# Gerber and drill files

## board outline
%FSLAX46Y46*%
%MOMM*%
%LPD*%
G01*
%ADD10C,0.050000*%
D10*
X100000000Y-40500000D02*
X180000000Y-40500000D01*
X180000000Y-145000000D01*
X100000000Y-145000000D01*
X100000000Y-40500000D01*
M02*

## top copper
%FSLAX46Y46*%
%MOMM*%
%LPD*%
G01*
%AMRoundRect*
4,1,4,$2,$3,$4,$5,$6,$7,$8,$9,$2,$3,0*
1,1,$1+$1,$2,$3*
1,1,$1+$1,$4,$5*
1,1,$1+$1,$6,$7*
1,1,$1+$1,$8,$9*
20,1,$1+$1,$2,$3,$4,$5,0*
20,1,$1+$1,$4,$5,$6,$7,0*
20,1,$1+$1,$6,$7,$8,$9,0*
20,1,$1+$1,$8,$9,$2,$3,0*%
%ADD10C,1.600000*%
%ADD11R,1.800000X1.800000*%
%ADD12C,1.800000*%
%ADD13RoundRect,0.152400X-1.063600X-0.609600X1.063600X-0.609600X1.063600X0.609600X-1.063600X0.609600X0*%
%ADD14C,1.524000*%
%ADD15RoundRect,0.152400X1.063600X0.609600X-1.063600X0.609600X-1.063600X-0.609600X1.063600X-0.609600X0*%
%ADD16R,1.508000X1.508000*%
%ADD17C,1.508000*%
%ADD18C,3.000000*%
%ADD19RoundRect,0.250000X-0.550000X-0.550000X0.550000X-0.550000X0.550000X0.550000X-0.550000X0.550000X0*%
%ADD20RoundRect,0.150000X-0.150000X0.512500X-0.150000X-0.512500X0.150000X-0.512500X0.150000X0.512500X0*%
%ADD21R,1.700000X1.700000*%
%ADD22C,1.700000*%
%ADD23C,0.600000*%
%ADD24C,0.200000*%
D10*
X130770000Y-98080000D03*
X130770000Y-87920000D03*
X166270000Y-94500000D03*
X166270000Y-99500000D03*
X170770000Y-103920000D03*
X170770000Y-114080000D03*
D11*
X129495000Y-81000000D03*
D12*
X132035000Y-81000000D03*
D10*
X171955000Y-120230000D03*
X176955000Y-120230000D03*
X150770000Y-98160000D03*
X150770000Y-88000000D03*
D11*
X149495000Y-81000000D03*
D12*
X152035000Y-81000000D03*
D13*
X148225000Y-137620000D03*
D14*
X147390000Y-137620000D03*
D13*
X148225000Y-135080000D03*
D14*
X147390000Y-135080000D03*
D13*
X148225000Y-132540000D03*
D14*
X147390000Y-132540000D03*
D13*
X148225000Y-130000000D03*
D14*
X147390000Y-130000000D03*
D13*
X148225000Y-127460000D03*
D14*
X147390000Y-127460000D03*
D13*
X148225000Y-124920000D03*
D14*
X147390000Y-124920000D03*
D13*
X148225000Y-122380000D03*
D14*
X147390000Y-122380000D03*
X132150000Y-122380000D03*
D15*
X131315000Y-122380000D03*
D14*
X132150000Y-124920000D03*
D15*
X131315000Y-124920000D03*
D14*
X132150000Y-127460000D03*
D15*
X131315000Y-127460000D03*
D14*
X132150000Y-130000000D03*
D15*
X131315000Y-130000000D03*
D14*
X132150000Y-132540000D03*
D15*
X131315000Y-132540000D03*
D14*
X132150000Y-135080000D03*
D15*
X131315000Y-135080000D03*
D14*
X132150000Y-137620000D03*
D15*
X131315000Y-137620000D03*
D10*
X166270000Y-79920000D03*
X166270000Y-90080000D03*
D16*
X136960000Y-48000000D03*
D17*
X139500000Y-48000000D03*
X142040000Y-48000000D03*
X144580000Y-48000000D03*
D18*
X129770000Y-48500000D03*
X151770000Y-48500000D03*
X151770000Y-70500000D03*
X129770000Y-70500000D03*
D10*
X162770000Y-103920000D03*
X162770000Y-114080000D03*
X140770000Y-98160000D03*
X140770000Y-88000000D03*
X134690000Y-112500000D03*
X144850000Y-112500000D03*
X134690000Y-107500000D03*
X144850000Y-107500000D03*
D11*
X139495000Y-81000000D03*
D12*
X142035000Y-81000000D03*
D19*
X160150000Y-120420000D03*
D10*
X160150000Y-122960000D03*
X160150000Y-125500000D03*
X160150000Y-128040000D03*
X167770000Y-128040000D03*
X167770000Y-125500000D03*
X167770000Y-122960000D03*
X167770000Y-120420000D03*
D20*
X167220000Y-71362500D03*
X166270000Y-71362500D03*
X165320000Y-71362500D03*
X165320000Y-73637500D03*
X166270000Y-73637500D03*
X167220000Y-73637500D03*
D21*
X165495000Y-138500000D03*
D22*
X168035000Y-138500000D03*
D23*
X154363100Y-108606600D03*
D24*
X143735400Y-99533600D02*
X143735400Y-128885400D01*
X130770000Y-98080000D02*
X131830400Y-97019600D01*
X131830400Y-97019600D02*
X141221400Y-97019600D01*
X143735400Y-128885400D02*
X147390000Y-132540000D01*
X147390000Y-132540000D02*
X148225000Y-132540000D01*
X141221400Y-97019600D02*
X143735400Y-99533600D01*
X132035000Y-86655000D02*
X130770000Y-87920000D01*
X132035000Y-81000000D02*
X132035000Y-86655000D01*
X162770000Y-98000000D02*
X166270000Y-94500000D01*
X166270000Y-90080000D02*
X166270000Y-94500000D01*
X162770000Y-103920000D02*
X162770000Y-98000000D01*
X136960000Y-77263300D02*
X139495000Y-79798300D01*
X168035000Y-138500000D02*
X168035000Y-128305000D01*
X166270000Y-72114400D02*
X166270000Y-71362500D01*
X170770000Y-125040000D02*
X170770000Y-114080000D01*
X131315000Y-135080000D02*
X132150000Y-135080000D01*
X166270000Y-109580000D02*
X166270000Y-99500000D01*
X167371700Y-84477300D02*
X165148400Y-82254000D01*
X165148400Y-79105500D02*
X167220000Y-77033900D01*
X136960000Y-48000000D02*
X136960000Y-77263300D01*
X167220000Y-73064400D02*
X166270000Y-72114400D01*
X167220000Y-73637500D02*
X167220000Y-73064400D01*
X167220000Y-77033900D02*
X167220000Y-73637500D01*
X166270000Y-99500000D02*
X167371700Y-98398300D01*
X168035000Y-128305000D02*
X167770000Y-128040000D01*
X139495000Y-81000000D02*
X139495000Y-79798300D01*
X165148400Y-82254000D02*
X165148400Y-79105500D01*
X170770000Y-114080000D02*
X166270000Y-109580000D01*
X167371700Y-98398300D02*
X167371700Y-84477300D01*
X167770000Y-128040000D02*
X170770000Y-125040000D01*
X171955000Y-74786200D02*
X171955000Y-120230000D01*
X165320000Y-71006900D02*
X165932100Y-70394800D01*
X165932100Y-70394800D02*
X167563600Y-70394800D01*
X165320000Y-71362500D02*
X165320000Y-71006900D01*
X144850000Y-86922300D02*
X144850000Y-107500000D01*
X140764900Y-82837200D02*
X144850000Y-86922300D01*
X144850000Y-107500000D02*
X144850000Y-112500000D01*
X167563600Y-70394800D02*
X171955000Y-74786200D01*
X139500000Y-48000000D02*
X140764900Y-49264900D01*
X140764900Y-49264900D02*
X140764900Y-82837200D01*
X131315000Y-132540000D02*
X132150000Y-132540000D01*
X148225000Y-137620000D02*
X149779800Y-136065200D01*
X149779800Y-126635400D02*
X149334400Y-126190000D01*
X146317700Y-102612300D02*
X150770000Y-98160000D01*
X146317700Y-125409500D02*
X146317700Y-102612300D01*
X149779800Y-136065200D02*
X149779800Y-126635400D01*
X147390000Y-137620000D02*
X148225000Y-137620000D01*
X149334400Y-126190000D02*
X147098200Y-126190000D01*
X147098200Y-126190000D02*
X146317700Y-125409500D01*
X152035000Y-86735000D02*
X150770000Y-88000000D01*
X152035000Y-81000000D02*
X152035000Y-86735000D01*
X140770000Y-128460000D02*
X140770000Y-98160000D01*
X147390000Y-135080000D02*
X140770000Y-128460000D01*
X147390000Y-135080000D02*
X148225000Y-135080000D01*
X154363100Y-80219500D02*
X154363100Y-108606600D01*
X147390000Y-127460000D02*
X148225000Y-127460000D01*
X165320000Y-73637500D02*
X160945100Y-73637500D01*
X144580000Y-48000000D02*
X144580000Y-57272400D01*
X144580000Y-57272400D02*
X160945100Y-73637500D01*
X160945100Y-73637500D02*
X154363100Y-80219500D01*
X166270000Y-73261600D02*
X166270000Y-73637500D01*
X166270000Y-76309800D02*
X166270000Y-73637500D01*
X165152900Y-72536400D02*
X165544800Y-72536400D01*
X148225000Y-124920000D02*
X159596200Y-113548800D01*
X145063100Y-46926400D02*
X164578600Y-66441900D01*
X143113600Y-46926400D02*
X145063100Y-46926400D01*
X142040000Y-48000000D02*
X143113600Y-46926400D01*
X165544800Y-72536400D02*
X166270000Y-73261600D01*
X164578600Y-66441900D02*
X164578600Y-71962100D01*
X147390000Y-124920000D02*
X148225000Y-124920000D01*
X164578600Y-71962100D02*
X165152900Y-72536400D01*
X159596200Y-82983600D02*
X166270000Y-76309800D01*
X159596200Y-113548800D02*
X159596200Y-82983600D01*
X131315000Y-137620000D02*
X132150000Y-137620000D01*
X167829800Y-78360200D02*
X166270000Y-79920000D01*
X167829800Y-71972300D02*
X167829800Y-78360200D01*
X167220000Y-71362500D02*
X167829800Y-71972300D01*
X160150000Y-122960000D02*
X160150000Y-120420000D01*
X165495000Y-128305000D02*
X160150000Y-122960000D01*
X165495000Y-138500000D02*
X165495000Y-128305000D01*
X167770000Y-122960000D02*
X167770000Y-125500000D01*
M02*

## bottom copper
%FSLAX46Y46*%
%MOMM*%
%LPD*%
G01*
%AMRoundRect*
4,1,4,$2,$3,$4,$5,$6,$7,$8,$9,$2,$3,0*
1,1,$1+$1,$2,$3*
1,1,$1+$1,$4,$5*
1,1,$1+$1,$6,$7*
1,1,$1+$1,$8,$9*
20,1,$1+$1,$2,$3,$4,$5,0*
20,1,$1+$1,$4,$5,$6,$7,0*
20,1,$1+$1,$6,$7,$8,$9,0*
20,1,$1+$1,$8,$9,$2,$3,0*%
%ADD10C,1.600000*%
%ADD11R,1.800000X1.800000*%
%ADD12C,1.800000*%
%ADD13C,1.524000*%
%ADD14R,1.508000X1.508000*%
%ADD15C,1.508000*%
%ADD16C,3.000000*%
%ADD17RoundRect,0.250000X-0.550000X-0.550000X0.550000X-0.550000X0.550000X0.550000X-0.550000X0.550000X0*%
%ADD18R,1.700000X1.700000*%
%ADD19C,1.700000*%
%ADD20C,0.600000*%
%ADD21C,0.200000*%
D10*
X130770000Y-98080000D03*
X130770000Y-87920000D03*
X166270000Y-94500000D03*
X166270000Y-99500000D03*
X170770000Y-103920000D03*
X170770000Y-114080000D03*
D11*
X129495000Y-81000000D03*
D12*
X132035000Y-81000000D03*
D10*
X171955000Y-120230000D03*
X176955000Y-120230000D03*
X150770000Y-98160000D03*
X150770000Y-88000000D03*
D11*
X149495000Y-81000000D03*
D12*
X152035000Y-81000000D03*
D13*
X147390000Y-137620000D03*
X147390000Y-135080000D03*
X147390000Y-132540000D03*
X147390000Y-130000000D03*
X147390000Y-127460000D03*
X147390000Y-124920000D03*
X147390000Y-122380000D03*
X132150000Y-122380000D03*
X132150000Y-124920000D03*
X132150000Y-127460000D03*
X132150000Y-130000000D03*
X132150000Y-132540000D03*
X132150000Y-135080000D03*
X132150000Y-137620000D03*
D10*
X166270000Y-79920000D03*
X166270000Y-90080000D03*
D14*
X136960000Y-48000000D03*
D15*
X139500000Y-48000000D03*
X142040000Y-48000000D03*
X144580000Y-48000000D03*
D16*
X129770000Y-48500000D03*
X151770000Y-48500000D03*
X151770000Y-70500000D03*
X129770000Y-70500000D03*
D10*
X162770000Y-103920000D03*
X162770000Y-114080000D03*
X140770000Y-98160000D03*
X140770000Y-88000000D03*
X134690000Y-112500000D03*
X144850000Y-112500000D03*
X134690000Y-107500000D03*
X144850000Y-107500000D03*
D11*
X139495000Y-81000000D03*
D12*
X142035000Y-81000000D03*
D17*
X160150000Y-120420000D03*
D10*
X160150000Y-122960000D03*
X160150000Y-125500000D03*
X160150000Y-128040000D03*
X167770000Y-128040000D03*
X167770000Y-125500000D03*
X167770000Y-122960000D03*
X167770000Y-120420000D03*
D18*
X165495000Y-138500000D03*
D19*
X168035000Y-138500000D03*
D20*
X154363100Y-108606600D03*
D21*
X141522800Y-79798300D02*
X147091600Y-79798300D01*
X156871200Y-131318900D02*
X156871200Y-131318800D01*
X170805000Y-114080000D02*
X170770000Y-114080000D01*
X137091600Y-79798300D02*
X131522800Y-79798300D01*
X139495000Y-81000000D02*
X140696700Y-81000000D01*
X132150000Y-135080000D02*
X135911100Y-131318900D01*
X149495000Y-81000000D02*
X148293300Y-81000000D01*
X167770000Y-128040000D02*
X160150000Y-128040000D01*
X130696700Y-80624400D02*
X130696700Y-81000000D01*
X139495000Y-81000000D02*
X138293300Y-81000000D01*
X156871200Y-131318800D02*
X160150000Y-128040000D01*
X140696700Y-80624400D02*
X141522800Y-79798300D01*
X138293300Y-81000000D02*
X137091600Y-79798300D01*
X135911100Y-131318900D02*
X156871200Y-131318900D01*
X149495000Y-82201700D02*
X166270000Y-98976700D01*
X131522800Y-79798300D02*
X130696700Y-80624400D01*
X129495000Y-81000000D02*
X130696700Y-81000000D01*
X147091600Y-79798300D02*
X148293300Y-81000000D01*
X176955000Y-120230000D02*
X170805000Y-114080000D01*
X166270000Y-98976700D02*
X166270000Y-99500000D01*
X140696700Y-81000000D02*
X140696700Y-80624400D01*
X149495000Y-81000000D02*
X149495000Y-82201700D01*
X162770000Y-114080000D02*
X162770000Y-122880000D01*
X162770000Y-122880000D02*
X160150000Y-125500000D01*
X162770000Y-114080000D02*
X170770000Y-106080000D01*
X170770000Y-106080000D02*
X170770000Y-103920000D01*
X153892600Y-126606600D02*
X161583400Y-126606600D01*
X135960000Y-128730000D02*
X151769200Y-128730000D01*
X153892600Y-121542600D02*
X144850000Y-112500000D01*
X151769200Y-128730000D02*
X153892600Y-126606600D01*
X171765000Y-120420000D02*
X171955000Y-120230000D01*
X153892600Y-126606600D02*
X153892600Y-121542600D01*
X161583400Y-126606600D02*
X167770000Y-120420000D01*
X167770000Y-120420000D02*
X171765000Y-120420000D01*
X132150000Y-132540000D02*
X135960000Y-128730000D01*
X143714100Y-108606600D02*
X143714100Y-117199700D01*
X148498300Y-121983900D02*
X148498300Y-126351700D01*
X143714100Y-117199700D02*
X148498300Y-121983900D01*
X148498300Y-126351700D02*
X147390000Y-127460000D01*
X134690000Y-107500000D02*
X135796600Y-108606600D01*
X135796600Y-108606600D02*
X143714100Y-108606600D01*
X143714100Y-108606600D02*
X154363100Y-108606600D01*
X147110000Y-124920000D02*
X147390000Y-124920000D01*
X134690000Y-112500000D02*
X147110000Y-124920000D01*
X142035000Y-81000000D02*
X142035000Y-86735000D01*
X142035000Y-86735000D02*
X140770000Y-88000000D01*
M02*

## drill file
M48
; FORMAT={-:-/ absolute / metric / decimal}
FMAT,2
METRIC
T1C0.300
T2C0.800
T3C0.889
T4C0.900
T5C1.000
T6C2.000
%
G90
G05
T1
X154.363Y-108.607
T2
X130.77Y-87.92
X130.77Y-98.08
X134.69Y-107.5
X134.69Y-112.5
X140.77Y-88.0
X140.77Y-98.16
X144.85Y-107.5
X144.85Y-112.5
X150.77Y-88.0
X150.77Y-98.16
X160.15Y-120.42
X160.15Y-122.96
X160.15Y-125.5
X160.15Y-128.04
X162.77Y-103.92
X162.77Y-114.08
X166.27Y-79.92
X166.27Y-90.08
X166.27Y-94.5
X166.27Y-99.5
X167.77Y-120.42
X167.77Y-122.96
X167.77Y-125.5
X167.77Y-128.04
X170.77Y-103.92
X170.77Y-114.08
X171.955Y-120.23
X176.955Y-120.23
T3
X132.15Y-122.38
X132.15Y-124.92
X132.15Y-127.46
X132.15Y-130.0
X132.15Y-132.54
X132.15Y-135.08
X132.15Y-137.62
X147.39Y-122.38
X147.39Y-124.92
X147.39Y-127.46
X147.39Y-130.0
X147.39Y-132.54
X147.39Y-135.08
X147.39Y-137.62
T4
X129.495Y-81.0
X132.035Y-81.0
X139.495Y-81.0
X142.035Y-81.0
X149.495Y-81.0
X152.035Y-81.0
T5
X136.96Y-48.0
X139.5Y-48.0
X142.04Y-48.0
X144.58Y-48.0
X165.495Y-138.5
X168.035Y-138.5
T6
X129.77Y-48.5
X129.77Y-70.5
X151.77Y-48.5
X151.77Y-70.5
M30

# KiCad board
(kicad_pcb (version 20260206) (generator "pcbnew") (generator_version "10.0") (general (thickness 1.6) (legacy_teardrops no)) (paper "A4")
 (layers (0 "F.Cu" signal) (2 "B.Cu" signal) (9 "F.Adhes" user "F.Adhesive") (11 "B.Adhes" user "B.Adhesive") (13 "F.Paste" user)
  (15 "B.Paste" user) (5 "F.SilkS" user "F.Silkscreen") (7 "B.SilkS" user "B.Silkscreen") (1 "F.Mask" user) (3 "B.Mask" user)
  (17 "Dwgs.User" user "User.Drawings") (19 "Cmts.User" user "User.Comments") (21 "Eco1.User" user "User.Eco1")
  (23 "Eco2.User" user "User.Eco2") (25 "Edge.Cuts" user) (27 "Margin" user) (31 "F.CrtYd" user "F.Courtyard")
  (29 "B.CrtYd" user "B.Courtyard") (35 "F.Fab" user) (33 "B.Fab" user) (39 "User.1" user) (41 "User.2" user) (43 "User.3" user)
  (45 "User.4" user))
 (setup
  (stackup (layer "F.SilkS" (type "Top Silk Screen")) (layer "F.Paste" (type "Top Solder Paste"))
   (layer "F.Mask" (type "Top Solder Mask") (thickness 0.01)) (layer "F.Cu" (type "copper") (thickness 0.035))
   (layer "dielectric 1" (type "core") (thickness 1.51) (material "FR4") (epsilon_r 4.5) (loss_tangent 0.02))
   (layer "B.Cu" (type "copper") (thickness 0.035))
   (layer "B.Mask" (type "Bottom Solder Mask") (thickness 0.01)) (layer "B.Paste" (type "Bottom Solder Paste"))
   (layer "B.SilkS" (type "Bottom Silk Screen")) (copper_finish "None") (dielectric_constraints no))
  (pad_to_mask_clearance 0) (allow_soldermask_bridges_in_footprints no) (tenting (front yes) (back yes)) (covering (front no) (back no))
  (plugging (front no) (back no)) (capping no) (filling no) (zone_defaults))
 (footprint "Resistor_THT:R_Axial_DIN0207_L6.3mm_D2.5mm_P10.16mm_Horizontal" (layer "F.Cu") (at 130.77 98.08 90)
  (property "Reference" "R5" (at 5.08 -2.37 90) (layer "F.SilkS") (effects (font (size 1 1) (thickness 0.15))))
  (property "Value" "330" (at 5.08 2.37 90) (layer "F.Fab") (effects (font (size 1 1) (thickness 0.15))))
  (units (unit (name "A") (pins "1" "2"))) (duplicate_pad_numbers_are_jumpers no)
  (pad "1" thru_hole circle (at 0 0 90) (size 1.6 1.6) (drill 0.8) (layers "*.Cu" "*.Mask") (remove_unused_layers no) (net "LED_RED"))
  (pad "2" thru_hole circle (at 10.16 0 90) (size 1.6 1.6) (drill 0.8) (layers "*.Cu" "*.Mask") (remove_unused_layers no) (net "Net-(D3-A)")))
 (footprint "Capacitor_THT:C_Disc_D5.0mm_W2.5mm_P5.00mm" (layer "F.Cu") (at 166.27 94.5 -90)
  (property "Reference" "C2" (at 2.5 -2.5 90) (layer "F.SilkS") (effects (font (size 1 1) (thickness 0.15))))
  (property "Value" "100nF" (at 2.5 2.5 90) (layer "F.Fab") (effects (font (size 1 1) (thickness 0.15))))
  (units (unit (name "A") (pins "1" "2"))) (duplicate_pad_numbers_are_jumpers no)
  (pad "1" thru_hole circle (at 0 0 270) (size 1.6 1.6) (drill 0.8) (layers "*.Cu" "*.Mask") (remove_unused_layers no) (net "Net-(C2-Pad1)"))
  (pad "2" thru_hole circle (at 5 0 270) (size 1.6 1.6) (drill 0.8) (layers "*.Cu" "*.Mask") (remove_unused_layers no) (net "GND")))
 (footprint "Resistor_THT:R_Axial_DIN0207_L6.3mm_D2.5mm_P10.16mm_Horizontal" (layer "F.Cu") (at 170.77 103.92 -90)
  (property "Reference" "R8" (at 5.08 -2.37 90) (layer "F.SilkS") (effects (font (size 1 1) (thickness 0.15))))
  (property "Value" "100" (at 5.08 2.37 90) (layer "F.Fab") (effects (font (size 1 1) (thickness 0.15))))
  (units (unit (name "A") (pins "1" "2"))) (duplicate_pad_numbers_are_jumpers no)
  (pad "1" thru_hole circle (at 0 0 270) (size 1.6 1.6) (drill 0.8) (layers "*.Cu" "*.Mask") (remove_unused_layers no) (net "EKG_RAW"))
  (pad "2" thru_hole circle (at 10.16 0 270) (size 1.6 1.6) (drill 0.8) (layers "*.Cu" "*.Mask") (remove_unused_layers no) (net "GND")))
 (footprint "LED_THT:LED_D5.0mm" (layer "F.Cu") (at 129.495 81)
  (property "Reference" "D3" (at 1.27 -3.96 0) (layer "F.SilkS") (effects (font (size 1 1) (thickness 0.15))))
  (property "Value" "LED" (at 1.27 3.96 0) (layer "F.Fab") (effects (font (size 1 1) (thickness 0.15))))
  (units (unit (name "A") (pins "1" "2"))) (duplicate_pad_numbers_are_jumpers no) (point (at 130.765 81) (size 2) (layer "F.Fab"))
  (pad "1" thru_hole rect (at 0 0) (size 1.8 1.8) (drill 0.9) (layers "*.Cu" "*.Mask") (remove_unused_layers no) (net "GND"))
  (pad "2" thru_hole circle (at 2.54 0) (size 1.8 1.8) (drill 0.9) (layers "*.Cu" "*.Mask") (remove_unused_layers no) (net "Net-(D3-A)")))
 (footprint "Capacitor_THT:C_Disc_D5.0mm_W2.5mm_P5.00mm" (layer "F.Cu") (at 171.955 120.23)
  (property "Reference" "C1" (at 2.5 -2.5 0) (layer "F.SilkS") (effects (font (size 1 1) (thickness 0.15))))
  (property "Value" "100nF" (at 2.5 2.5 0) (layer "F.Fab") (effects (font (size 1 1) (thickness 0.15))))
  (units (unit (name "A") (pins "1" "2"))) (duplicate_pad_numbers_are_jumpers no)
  (pad "1" thru_hole circle (at 0 0) (size 1.6 1.6) (drill 0.8) (layers "*.Cu" "*.Mask") (remove_unused_layers no) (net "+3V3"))
  (pad "2" thru_hole circle (at 5 0) (size 1.6 1.6) (drill 0.8) (layers "*.Cu" "*.Mask") (remove_unused_layers no) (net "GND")))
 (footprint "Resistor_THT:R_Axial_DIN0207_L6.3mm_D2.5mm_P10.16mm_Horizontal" (layer "F.Cu") (at 150.77 98.16 90)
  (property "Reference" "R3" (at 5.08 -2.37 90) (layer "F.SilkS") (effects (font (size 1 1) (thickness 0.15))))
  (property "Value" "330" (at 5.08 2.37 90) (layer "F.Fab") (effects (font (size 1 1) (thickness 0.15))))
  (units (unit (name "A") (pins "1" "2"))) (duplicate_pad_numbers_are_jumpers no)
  (pad "1" thru_hole circle (at 0 0 90) (size 1.6 1.6) (drill 0.8) (layers "*.Cu" "*.Mask") (remove_unused_layers no) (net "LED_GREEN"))
  (pad "2" thru_hole circle (at 10.16 0 90) (size 1.6 1.6) (drill 0.8) (layers "*.Cu" "*.Mask") (remove_unused_layers no) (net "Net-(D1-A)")))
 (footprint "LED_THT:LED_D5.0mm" (layer "F.Cu") (at 149.495 81)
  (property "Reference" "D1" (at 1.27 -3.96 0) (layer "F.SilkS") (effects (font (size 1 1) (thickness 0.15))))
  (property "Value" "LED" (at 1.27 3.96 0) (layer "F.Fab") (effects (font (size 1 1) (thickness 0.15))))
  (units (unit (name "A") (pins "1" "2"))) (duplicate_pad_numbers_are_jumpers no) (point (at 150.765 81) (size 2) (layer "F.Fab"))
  (pad "1" thru_hole rect (at 0 0) (size 1.8 1.8) (drill 0.9) (layers "*.Cu" "*.Mask") (remove_unused_layers no) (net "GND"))
  (pad "2" thru_hole circle (at 2.54 0) (size 1.8 1.8) (drill 0.9) (layers "*.Cu" "*.Mask") (remove_unused_layers no) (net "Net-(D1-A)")))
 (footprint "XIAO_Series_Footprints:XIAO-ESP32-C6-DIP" (layer "F.Cu") (at 139.77 130 -90)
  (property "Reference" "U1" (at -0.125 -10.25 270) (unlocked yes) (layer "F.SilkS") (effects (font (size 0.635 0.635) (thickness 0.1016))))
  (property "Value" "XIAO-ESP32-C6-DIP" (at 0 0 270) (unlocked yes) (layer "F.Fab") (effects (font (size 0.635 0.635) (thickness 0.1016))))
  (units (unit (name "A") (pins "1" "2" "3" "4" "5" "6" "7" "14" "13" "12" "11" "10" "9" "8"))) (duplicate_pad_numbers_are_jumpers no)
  (pad "1" smd roundrect (at 7.62 -8.455) (size 2.432 1.524) (layers "F.Cu" "F.Mask") (roundrect_rratio 0.1) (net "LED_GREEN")
   (thermal_bridge_angle 45))
  (pad "1" thru_hole circle (at 7.62 -7.62) (size 1.524 1.524) (drill 0.889) (layers "*.Cu" "*.Mask") (remove_unused_layers no)
   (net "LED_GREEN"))
  (pad "2" smd roundrect (at 5.08 -8.455) (size 2.432 1.524) (layers "F.Cu" "F.Mask") (roundrect_rratio 0.1) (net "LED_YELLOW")
   (thermal_bridge_angle 45))
  (pad "2" thru_hole circle (at 5.08 -7.62) (size 1.524 1.524) (drill 0.889) (layers "*.Cu" "*.Mask") (remove_unused_layers no)
   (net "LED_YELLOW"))
  (pad "3" smd roundrect (at 2.54 -8.455) (size 2.432 1.524) (layers "F.Cu" "F.Mask") (roundrect_rratio 0.1) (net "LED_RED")
   (thermal_bridge_angle 45))
  (pad "3" thru_hole circle (at 2.54 -7.62) (size 1.524 1.524) (drill 0.889) (layers "*.Cu" "*.Mask") (remove_unused_layers no)
   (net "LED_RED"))
  (pad "4" smd roundrect (at 0 -8.455) (size 2.432 1.524) (layers "F.Cu" "F.Mask") (roundrect_rratio 0.1)
   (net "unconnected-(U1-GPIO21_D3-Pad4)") (thermal_bridge_angle 45))
  (pad "4" thru_hole circle (at 0 -7.62) (size 1.524 1.524) (drill 0.889) (layers "*.Cu" "*.Mask") (remove_unused_layers no)
   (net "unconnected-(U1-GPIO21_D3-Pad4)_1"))
  (pad "5" smd roundrect (at -2.54 -8.455) (size 2.432 1.524) (layers "F.Cu" "F.Mask") (roundrect_rratio 0.1) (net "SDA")
   (thermal_bridge_angle 45))
  (pad "5" thru_hole circle (at -2.54 -7.62) (size 1.524 1.524) (drill 0.889) (layers "*.Cu" "*.Mask") (remove_unused_layers no) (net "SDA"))
  (pad "6" smd roundrect (at -5.08 -8.455) (size 2.432 1.524) (layers "F.Cu" "F.Mask") (roundrect_rratio 0.1) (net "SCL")
   (thermal_bridge_angle 45))
  (pad "6" thru_hole circle (at -5.08 -7.62) (size 1.524 1.524) (drill 0.889) (layers "*.Cu" "*.Mask") (remove_unused_layers no) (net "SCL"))
  (pad "7" smd roundrect (at -7.62 -8.455) (size 2.432 1.524) (layers "F.Cu" "F.Mask") (roundrect_rratio 0.1)
   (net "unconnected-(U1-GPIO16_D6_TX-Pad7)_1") (thermal_bridge_angle 45))
  (pad "7" thru_hole circle (at -7.62 -7.62) (size 1.524 1.524) (drill 0.889) (layers "*.Cu" "*.Mask") (remove_unused_layers no)
   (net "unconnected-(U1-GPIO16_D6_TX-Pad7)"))
  (pad "8" thru_hole circle (at -7.62 7.62 180) (size 1.524 1.524) (drill 0.889) (layers "*.Cu" "*.Mask") (remove_unused_layers no)
   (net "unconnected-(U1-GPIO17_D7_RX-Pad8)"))
  (pad "8" smd roundrect (at -7.62 8.455 180) (size 2.432 1.524) (layers "F.Cu" "F.Mask") (roundrect_rratio 0.1)
   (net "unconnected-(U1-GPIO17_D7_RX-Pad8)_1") (thermal_bridge_angle 45))
  (pad "9" thru_hole circle (at -5.08 7.62 180) (size 1.524 1.524) (drill 0.889) (layers "*.Cu" "*.Mask") (remove_unused_layers no)
   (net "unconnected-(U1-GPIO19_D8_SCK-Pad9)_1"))
  (pad "9" smd roundrect (at -5.08 8.455 180) (size 2.432 1.524) (layers "F.Cu" "F.Mask") (roundrect_rratio 0.1)
   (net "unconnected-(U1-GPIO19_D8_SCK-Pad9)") (thermal_bridge_angle 45))
  (pad "10" thru_hole circle (at -2.54 7.62 180) (size 1.524 1.524) (drill 0.889) (layers "*.Cu" "*.Mask") (remove_unused_layers no)
   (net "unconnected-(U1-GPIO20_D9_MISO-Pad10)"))
  (pad "10" smd roundrect (at -2.54 8.455 180) (size 2.432 1.524) (layers "F.Cu" "F.Mask") (roundrect_rratio 0.1)
   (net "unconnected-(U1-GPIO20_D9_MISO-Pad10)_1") (thermal_bridge_angle 45))
  (pad "11" thru_hole circle (at 0 7.62 180) (size 1.524 1.524) (drill 0.889) (layers "*.Cu" "*.Mask") (remove_unused_layers no)
   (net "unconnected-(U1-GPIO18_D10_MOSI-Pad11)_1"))
  (pad "11" smd roundrect (at 0 8.455 180) (size 2.432 1.524) (layers "F.Cu" "F.Mask") (roundrect_rratio 0.1)
   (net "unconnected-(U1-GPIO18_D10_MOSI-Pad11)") (thermal_bridge_angle 45))
  (pad "12" thru_hole circle (at 2.54 7.62 180) (size 1.524 1.524) (drill 0.889) (layers "*.Cu" "*.Mask") (remove_unused_layers no)
   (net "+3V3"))
  (pad "12" smd roundrect (at 2.54 8.455 180) (size 2.432 1.524) (layers "F.Cu" "F.Mask") (roundrect_rratio 0.1) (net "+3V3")
   (thermal_bridge_angle 45))
  (pad "13" thru_hole circle (at 5.08 7.62 180) (size 1.524 1.524) (drill 0.889) (layers "*.Cu" "*.Mask") (remove_unused_layers no)
   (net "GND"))
  (pad "13" smd roundrect (at 5.08 8.455 180) (size 2.432 1.524) (layers "F.Cu" "F.Mask") (roundrect_rratio 0.1) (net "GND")
   (thermal_bridge_angle 45))
  (pad "14" thru_hole circle (at 7.62 7.62 180) (size 1.524 1.524) (drill 0.889) (layers "*.Cu" "*.Mask") (remove_unused_layers no)
   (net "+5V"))
  (pad "14" smd roundrect (at 7.62 8.455 180) (size 2.432 1.524) (layers "F.Cu" "F.Mask") (roundrect_rratio 0.1) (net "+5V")
   (thermal_bridge_angle 45)))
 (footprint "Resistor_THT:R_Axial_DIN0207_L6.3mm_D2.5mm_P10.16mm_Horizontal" (layer "F.Cu") (at 166.27 79.92 -90)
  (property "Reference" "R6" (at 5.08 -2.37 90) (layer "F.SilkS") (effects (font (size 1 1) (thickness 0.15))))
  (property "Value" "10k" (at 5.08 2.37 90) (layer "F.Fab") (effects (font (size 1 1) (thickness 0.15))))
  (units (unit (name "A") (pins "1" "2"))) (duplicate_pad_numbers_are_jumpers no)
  (pad "1" thru_hole circle (at 0 0 270) (size 1.6 1.6) (drill 0.8) (layers "*.Cu" "*.Mask") (remove_unused_layers no) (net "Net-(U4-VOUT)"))
  (pad "2" thru_hole circle (at 10.16 0 270) (size 1.6 1.6) (drill 0.8) (layers "*.Cu" "*.Mask") (remove_unused_layers no)
   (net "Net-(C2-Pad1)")))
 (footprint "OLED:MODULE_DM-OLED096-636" (layer "F.Cu") (at 140.77 59.5)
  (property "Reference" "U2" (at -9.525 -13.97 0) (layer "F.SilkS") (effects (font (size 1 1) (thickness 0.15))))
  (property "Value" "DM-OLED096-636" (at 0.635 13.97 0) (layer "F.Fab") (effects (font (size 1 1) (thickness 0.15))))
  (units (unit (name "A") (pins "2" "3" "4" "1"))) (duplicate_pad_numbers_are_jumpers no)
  (pad "1" thru_hole rect (at -3.81 -11.5) (size 1.508 1.508) (drill 1) (layers "*.Cu" "*.Mask") (remove_unused_layers no) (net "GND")
   (solder_mask_margin 0.102))
  (pad "2" thru_hole circle (at -1.27 -11.5) (size 1.508 1.508) (drill 1) (layers "*.Cu" "*.Mask") (remove_unused_layers no) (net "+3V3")
   (solder_mask_margin 0.102))
  (pad "3" thru_hole circle (at 1.27 -11.5) (size 1.508 1.508) (drill 1) (layers "*.Cu" "*.Mask") (remove_unused_layers no) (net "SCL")
   (solder_mask_margin 0.102))
  (pad "4" thru_hole circle (at 3.81 -11.5) (size 1.508 1.508) (drill 1) (layers "*.Cu" "*.Mask") (remove_unused_layers no) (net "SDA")
   (solder_mask_margin 0.102))
  (pad "S1" thru_hole circle (at -11 -11) (size 3 3) (drill 2) (layers "*.Cu" "*.Mask") (remove_unused_layers no) (solder_mask_margin 0.102))
  (pad "S2" thru_hole circle (at 11 -11) (size 3 3) (drill 2) (layers "*.Cu" "*.Mask") (remove_unused_layers no) (solder_mask_margin 0.102))
  (pad "S3" thru_hole circle (at 11 11) (size 3 3) (drill 2) (layers "*.Cu" "*.Mask") (remove_unused_layers no) (solder_mask_margin 0.102))
  (pad "S4" thru_hole circle (at -11 11) (size 3 3) (drill 2) (layers "*.Cu" "*.Mask") (remove_unused_layers no) (solder_mask_margin 0.102)))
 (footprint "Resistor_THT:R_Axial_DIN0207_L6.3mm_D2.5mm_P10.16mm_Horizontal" (layer "F.Cu") (at 162.77 103.92 -90)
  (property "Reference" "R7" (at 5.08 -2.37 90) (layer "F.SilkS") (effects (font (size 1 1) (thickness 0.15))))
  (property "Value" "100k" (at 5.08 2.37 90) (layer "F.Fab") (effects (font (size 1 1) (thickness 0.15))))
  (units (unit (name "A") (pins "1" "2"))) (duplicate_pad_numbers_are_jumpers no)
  (pad "1" thru_hole circle (at 0 0 270) (size 1.6 1.6) (drill 0.8) (layers "*.Cu" "*.Mask") (remove_unused_layers no) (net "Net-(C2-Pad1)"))
  (pad "2" thru_hole circle (at 10.16 0 270) (size 1.6 1.6) (drill 0.8) (layers "*.Cu" "*.Mask") (remove_unused_layers no) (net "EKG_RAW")))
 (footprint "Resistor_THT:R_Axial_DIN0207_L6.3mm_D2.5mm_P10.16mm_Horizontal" (layer "F.Cu") (at 140.77 98.16 90)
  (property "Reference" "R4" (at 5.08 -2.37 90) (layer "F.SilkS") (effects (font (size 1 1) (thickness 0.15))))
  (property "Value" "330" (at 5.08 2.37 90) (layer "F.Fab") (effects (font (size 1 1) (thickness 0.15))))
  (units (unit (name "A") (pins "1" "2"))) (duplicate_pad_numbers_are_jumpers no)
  (pad "1" thru_hole circle (at 0 0 90) (size 1.6 1.6) (drill 0.8) (layers "*.Cu" "*.Mask") (remove_unused_layers no) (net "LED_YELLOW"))
  (pad "2" thru_hole circle (at 10.16 0 90) (size 1.6 1.6) (drill 0.8) (layers "*.Cu" "*.Mask") (remove_unused_layers no) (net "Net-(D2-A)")))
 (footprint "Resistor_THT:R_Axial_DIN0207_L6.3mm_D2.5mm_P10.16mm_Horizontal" (layer "F.Cu") (at 134.69 112.5)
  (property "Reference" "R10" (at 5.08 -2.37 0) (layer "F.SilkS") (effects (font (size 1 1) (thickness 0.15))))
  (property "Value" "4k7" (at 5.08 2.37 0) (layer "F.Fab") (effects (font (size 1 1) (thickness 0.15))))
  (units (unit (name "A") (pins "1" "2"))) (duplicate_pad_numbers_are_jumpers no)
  (pad "1" thru_hole circle (at 0 0) (size 1.6 1.6) (drill 0.8) (layers "*.Cu" "*.Mask") (remove_unused_layers no) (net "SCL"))
  (pad "2" thru_hole circle (at 10.16 0) (size 1.6 1.6) (drill 0.8) (layers "*.Cu" "*.Mask") (remove_unused_layers no) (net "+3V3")))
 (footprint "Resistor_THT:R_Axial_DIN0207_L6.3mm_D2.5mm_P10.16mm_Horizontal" (layer "F.Cu") (at 134.69 107.5)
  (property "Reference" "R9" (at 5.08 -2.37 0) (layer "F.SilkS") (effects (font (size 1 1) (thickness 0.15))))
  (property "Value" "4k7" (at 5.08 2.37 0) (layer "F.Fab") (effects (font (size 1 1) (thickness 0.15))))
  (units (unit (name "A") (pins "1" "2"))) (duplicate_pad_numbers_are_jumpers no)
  (pad "1" thru_hole circle (at 0 0) (size 1.6 1.6) (drill 0.8) (layers "*.Cu" "*.Mask") (remove_unused_layers no) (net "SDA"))
  (pad "2" thru_hole circle (at 10.16 0) (size 1.6 1.6) (drill 0.8) (layers "*.Cu" "*.Mask") (remove_unused_layers no) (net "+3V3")))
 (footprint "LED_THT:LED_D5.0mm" (layer "F.Cu") (at 139.495 81)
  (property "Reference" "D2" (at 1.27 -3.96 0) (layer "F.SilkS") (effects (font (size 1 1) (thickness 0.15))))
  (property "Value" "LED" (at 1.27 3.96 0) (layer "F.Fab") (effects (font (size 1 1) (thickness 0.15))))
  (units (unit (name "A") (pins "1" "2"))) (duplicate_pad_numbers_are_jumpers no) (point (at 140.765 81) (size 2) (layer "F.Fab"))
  (pad "1" thru_hole rect (at 0 0) (size 1.8 1.8) (drill 0.9) (layers "*.Cu" "*.Mask") (remove_unused_layers no) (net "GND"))
  (pad "2" thru_hole circle (at 2.54 0) (size 1.8 1.8) (drill 0.9) (layers "*.Cu" "*.Mask") (remove_unused_layers no) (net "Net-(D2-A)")))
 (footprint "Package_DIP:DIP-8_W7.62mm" (layer "F.Cu") (at 160.15 120.42)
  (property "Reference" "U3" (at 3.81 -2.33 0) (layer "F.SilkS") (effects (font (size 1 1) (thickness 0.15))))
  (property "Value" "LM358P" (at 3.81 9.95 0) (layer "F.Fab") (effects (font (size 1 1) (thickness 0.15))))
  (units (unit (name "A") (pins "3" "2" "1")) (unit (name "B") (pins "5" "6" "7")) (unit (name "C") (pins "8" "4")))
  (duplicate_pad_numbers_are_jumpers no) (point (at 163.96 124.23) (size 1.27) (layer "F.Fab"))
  (pad "1" thru_hole roundrect (at 0 0) (size 1.6 1.6) (drill 0.8) (layers "*.Cu" "*.Mask") (remove_unused_layers no)
   (roundrect_rratio 0.15625) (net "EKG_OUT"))
  (pad "2" thru_hole circle (at 0 2.54) (size 1.6 1.6) (drill 0.8) (layers "*.Cu" "*.Mask") (remove_unused_layers no) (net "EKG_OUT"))
  (pad "3" thru_hole circle (at 0 5.08) (size 1.6 1.6) (drill 0.8) (layers "*.Cu" "*.Mask") (remove_unused_layers no) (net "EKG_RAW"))
  (pad "4" thru_hole circle (at 0 7.62) (size 1.6 1.6) (drill 0.8) (layers "*.Cu" "*.Mask") (remove_unused_layers no) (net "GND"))
  (pad "5" thru_hole circle (at 7.62 7.62) (size 1.6 1.6) (drill 0.8) (layers "*.Cu" "*.Mask") (remove_unused_layers no) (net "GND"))
  (pad "6" thru_hole circle (at 7.62 5.08) (size 1.6 1.6) (drill 0.8) (layers "*.Cu" "*.Mask") (remove_unused_layers no)
   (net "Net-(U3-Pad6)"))
  (pad "7" thru_hole circle (at 7.62 2.54) (size 1.6 1.6) (drill 0.8) (layers "*.Cu" "*.Mask") (remove_unused_layers no)
   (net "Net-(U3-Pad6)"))
  (pad "8" thru_hole circle (at 7.62 0) (size 1.6 1.6) (drill 0.8) (layers "*.Cu" "*.Mask") (remove_unused_layers no) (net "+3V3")))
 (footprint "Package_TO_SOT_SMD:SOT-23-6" (layer "F.Cu") (at 166.27 72.5 -90)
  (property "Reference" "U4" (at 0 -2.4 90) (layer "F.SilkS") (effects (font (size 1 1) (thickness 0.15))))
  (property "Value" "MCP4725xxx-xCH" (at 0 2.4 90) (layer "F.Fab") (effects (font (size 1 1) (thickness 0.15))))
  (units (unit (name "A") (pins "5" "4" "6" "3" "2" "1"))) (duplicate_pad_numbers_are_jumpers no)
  (pad "1" smd roundrect (at -1.1375 -0.95 270) (size 1.325 0.6) (layers "F.Cu" "F.Mask" "F.Paste") (roundrect_rratio 0.25)
   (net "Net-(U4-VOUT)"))
  (pad "2" smd roundrect (at -1.1375 0 270) (size 1.325 0.6) (layers "F.Cu" "F.Mask" "F.Paste") (roundrect_rratio 0.25) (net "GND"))
  (pad "3" smd roundrect (at -1.1375 0.95 270) (size 1.325 0.6) (layers "F.Cu" "F.Mask" "F.Paste") (roundrect_rratio 0.25) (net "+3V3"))
  (pad "4" smd roundrect (at 1.1375 0.95 270) (size 1.325 0.6) (layers "F.Cu" "F.Mask" "F.Paste") (roundrect_rratio 0.25) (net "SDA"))
  (pad "5" smd roundrect (at 1.1375 0 270) (size 1.325 0.6) (layers "F.Cu" "F.Mask" "F.Paste") (roundrect_rratio 0.25) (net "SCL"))
  (pad "6" smd roundrect (at 1.1375 -0.95 270) (size 1.325 0.6) (layers "F.Cu" "F.Mask" "F.Paste") (roundrect_rratio 0.25) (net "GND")))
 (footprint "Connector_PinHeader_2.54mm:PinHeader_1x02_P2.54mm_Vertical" (layer "F.Cu") (at 165.495 138.5 90)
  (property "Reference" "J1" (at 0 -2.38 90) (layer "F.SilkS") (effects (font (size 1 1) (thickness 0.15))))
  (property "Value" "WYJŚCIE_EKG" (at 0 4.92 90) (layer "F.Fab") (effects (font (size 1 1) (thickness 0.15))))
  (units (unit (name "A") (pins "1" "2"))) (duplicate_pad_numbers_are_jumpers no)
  (pad "1" thru_hole rect (at 0 0 90) (size 1.7 1.7) (drill 1) (layers "*.Cu" "*.Mask") (remove_unused_layers no) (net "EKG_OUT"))
  (pad "2" thru_hole circle (at 0 2.54 90) (size 1.7 1.7) (drill 1) (layers "*.Cu" "*.Mask") (remove_unused_layers no) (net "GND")))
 (gr_rect (start 100 40.5) (end 180 145) (stroke (width 0.05) (type default)) (fill no) (layer "Edge.Cuts"))
 (segment (start 143.7354 99.5336) (end 143.7354 128.8854) (width 0.2) (layer "F.Cu") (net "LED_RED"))
 (segment (start 130.77 98.08) (end 131.8304 97.0196) (width 0.2) (layer "F.Cu") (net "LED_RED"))
 (segment (start 131.8304 97.0196) (end 141.2214 97.0196) (width 0.2) (layer "F.Cu") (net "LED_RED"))
 (segment (start 143.7354 128.8854) (end 147.39 132.54) (width 0.2) (layer "F.Cu") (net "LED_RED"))
 (segment (start 147.39 132.54) (end 148.225 132.54) (width 0.2) (layer "F.Cu") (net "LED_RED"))
 (segment (start 141.2214 97.0196) (end 143.7354 99.5336) (width 0.2) (layer "F.Cu") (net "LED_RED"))
 (segment (start 132.035 86.655) (end 130.77 87.92) (width 0.2) (layer "F.Cu") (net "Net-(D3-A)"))
 (segment (start 132.035 81) (end 132.035 86.655) (width 0.2) (layer "F.Cu") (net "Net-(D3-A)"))
 (segment (start 162.77 98) (end 166.27 94.5) (width 0.2) (layer "F.Cu") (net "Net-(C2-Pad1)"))
 (segment (start 166.27 90.08) (end 166.27 94.5) (width 0.2) (layer "F.Cu") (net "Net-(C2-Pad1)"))
 (segment (start 162.77 103.92) (end 162.77 98) (width 0.2) (layer "F.Cu") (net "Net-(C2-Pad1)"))
 (segment (start 136.96 77.2633) (end 139.495 79.7983) (width 0.2) (layer "F.Cu") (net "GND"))
 (segment (start 168.035 138.5) (end 168.035 128.305) (width 0.2) (layer "F.Cu") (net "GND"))
 (segment (start 166.27 72.1144) (end 166.27 71.3625) (width 0.2) (layer "F.Cu") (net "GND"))
 (segment (start 170.77 125.04) (end 170.77 114.08) (width 0.2) (layer "F.Cu") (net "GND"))
 (segment (start 131.315 135.08) (end 132.15 135.08) (width 0.2) (layer "F.Cu") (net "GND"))
 (segment (start 166.27 109.58) (end 166.27 99.5) (width 0.2) (layer "F.Cu") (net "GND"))
 (segment (start 167.3717 84.4773) (end 165.1484 82.254) (width 0.2) (layer "F.Cu") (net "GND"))
 (segment (start 165.1484 79.1055) (end 167.22 77.0339) (width 0.2) (layer "F.Cu") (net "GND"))
 (segment (start 136.96 48) (end 136.96 77.2633) (width 0.2) (layer "F.Cu") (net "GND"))
 (segment (start 167.22 73.0644) (end 166.27 72.1144) (width 0.2) (layer "F.Cu") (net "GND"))
 (segment (start 167.22 73.6375) (end 167.22 73.0644) (width 0.2) (layer "F.Cu") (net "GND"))
 (segment (start 167.22 77.0339) (end 167.22 73.6375) (width 0.2) (layer "F.Cu") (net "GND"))
 (segment (start 166.27 99.5) (end 167.3717 98.3983) (width 0.2) (layer "F.Cu") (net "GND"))
 (segment (start 168.035 128.305) (end 167.77 128.04) (width 0.2) (layer "F.Cu") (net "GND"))
 (segment (start 139.495 81) (end 139.495 79.7983) (width 0.2) (layer "F.Cu") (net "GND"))
 (segment (start 165.1484 82.254) (end 165.1484 79.1055) (width 0.2) (layer "F.Cu") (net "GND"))
 (segment (start 170.77 114.08) (end 166.27 109.58) (width 0.2) (layer "F.Cu") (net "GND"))
 (segment (start 167.3717 98.3983) (end 167.3717 84.4773) (width 0.2) (layer "F.Cu") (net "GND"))
 (segment (start 167.77 128.04) (end 170.77 125.04) (width 0.2) (layer "F.Cu") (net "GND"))
 (segment (start 141.5228 79.7983) (end 147.0916 79.7983) (width 0.2) (layer "B.Cu") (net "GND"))
 (segment (start 156.8712 131.3189) (end 156.8712 131.3188) (width 0.2) (layer "B.Cu") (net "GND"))
 (segment (start 170.805 114.08) (end 170.77 114.08) (width 0.2) (layer "B.Cu") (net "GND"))
 (segment (start 137.0916 79.7983) (end 131.5228 79.7983) (width 0.2) (layer "B.Cu") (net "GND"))
 (segment (start 139.495 81) (end 140.6967 81) (width 0.2) (layer "B.Cu") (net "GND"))
 (segment (start 132.15 135.08) (end 135.9111 131.3189) (width 0.2) (layer "B.Cu") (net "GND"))
 (segment (start 149.495 81) (end 148.2933 81) (width 0.2) (layer "B.Cu") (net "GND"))
 (segment (start 167.77 128.04) (end 160.15 128.04) (width 0.2) (layer "B.Cu") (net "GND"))
 (segment (start 130.6967 80.6244) (end 130.6967 81) (width 0.2) (layer "B.Cu") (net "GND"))
 (segment (start 139.495 81) (end 138.2933 81) (width 0.2) (layer "B.Cu") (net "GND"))
 (segment (start 156.8712 131.3188) (end 160.15 128.04) (width 0.2) (layer "B.Cu") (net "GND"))
 (segment (start 140.6967 80.6244) (end 141.5228 79.7983) (width 0.2) (layer "B.Cu") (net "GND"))
 (segment (start 138.2933 81) (end 137.0916 79.7983) (width 0.2) (layer "B.Cu") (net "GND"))
 (segment (start 135.9111 131.3189) (end 156.8712 131.3189) (width 0.2) (layer "B.Cu") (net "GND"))
 (segment (start 149.495 82.2017) (end 166.27 98.9767) (width 0.2) (layer "B.Cu") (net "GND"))
 (segment (start 131.5228 79.7983) (end 130.6967 80.6244) (width 0.2) (layer "B.Cu") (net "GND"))
 (segment (start 129.495 81) (end 130.6967 81) (width 0.2) (layer "B.Cu") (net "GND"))
 (segment (start 147.0916 79.7983) (end 148.2933 81) (width 0.2) (layer "B.Cu") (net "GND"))
 (segment (start 176.955 120.23) (end 170.805 114.08) (width 0.2) (layer "B.Cu") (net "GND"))
 (segment (start 166.27 98.9767) (end 166.27 99.5) (width 0.2) (layer "B.Cu") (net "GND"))
 (segment (start 140.6967 81) (end 140.6967 80.6244) (width 0.2) (layer "B.Cu") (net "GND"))
 (segment (start 149.495 81) (end 149.495 82.2017) (width 0.2) (layer "B.Cu") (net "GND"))
 (segment (start 162.77 114.08) (end 162.77 122.88) (width 0.2) (layer "B.Cu") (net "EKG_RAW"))
 (segment (start 162.77 122.88) (end 160.15 125.5) (width 0.2) (layer "B.Cu") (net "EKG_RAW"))
 (segment (start 162.77 114.08) (end 170.77 106.08) (width 0.2) (layer "B.Cu") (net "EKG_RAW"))
 (segment (start 170.77 106.08) (end 170.77 103.92) (width 0.2) (layer "B.Cu") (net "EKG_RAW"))
 (segment (start 171.955 74.7862) (end 171.955 120.23) (width 0.2) (layer "F.Cu") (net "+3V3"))
 (segment (start 165.32 71.0069) (end 165.9321 70.3948) (width 0.2) (layer "F.Cu") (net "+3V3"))
 (segment (start 165.9321 70.3948) (end 167.5636 70.3948) (width 0.2) (layer "F.Cu") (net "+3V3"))
 (segment (start 165.32 71.3625) (end 165.32 71.0069) (width 0.2) (layer "F.Cu") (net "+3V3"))
 (segment (start 144.85 86.9223) (end 144.85 107.5) (width 0.2) (layer "F.Cu") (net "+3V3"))
 (segment (start 140.7649 82.8372) (end 144.85 86.9223) (width 0.2) (layer "F.Cu") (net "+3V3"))
 (segment (start 144.85 107.5) (end 144.85 112.5) (width 0.2) (layer "F.Cu") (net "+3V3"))
 (segment (start 167.5636 70.3948) (end 171.955 74.7862) (width 0.2) (layer "F.Cu") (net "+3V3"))
 (segment (start 139.5 48) (end 140.7649 49.2649) (width 0.2) (layer "F.Cu") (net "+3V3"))
 (segment (start 140.7649 49.2649) (end 140.7649 82.8372) (width 0.2) (layer "F.Cu") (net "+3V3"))
 (segment (start 131.315 132.54) (end 132.15 132.54) (width 0.2) (layer "F.Cu") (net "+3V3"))
 (segment (start 153.8926 126.6066) (end 161.5834 126.6066) (width 0.2) (layer "B.Cu") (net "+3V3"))
 (segment (start 135.96 128.73) (end 151.7692 128.73) (width 0.2) (layer "B.Cu") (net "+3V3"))
 (segment (start 153.8926 121.5426) (end 144.85 112.5) (width 0.2) (layer "B.Cu") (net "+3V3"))
 (segment (start 151.7692 128.73) (end 153.8926 126.6066) (width 0.2) (layer "B.Cu") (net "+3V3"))
 (segment (start 171.765 120.42) (end 171.955 120.23) (width 0.2) (layer "B.Cu") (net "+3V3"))
 (segment (start 153.8926 126.6066) (end 153.8926 121.5426) (width 0.2) (layer "B.Cu") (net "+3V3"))
 (segment (start 161.5834 126.6066) (end 167.77 120.42) (width 0.2) (layer "B.Cu") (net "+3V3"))
 (segment (start 167.77 120.42) (end 171.765 120.42) (width 0.2) (layer "B.Cu") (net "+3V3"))
 (segment (start 132.15 132.54) (end 135.96 128.73) (width 0.2) (layer "B.Cu") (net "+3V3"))
 (segment (start 148.225 137.62) (end 149.7798 136.0652) (width 0.2) (layer "F.Cu") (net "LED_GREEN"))
 (segment (start 149.7798 126.6354) (end 149.3344 126.19) (width 0.2) (layer "F.Cu") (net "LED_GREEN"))
 (segment (start 146.3177 102.6123) (end 150.77 98.16) (width 0.2) (layer "F.Cu") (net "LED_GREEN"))
 (segment (start 146.3177 125.4095) (end 146.3177 102.6123) (width 0.2) (layer "F.Cu") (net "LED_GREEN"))
 (segment (start 149.7798 136.0652) (end 149.7798 126.6354) (width 0.2) (layer "F.Cu") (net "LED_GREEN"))
 (segment (start 147.39 137.62) (end 148.225 137.62) (width 0.2) (layer "F.Cu") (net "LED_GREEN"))
 (segment (start 149.3344 126.19) (end 147.0982 126.19) (width 0.2) (layer "F.Cu") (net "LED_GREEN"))
 (segment (start 147.0982 126.19) (end 146.3177 125.4095) (width 0.2) (layer "F.Cu") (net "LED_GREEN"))
 (segment (start 152.035 86.735) (end 150.77 88) (width 0.2) (layer "F.Cu") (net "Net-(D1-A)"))
 (segment (start 152.035 81) (end 152.035 86.735) (width 0.2) (layer "F.Cu") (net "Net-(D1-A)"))
 (segment (start 140.77 128.46) (end 140.77 98.16) (width 0.2) (layer "F.Cu") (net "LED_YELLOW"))
 (segment (start 147.39 135.08) (end 140.77 128.46) (width 0.2) (layer "F.Cu") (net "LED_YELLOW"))
 (segment (start 147.39 135.08) (end 148.225 135.08) (width 0.2) (layer "F.Cu") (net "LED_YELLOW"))
 (segment (start 154.3631 80.2195) (end 154.3631 108.6066) (width 0.2) (layer "F.Cu") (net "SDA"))
 (segment (start 147.39 127.46) (end 148.225 127.46) (width 0.2) (layer "F.Cu") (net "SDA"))
 (segment (start 165.32 73.6375) (end 160.9451 73.6375) (width 0.2) (layer "F.Cu") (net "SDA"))
 (segment (start 144.58 48) (end 144.58 57.2724) (width 0.2) (layer "F.Cu") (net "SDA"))
 (segment (start 144.58 57.2724) (end 160.9451 73.6375) (width 0.2) (layer "F.Cu") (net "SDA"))
 (segment (start 160.9451 73.6375) (end 154.3631 80.2195) (width 0.2) (layer "F.Cu") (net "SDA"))
 (via (at 154.3631 108.6066) (size 0.6) (drill 0.3) (layers "F.Cu" "B.Cu") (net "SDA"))
 (segment (start 143.7141 108.6066) (end 143.7141 117.1997) (width 0.2) (layer "B.Cu") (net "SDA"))
 (segment (start 148.4983 121.9839) (end 148.4983 126.3517) (width 0.2) (layer "B.Cu") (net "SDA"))
 (segment (start 143.7141 117.1997) (end 148.4983 121.9839) (width 0.2) (layer "B.Cu") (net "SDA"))
 (segment (start 148.4983 126.3517) (end 147.39 127.46) (width 0.2) (layer "B.Cu") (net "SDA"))
 (segment (start 134.69 107.5) (end 135.7966 108.6066) (width 0.2) (layer "B.Cu") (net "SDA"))
 (segment (start 135.7966 108.6066) (end 143.7141 108.6066) (width 0.2) (layer "B.Cu") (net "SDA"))
 (segment (start 143.7141 108.6066) (end 154.3631 108.6066) (width 0.2) (layer "B.Cu") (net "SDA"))
 (segment (start 166.27 73.2616) (end 166.27 73.6375) (width 0.2) (layer "F.Cu") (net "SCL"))
 (segment (start 166.27 76.3098) (end 166.27 73.6375) (width 0.2) (layer "F.Cu") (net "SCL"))
 (segment (start 165.1529 72.5364) (end 165.5448 72.5364) (width 0.2) (layer "F.Cu") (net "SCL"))
 (segment (start 148.225 124.92) (end 159.5962 113.5488) (width 0.2) (layer "F.Cu") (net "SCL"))
 (segment (start 145.0631 46.9264) (end 164.5786 66.4419) (width 0.2) (layer "F.Cu") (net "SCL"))
 (segment (start 143.1136 46.9264) (end 145.0631 46.9264) (width 0.2) (layer "F.Cu") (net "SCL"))
 (segment (start 142.04 48) (end 143.1136 46.9264) (width 0.2) (layer "F.Cu") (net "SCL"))
 (segment (start 165.5448 72.5364) (end 166.27 73.2616) (width 0.2) (layer "F.Cu") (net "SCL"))
 (segment (start 164.5786 66.4419) (end 164.5786 71.9621) (width 0.2) (layer "F.Cu") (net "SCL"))
 (segment (start 147.39 124.92) (end 148.225 124.92) (width 0.2) (layer "F.Cu") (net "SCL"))
 (segment (start 164.5786 71.9621) (end 165.1529 72.5364) (width 0.2) (layer "F.Cu") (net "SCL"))
 (segment (start 159.5962 82.9836) (end 166.27 76.3098) (width 0.2) (layer "F.Cu") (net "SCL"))
 (segment (start 159.5962 113.5488) (end 159.5962 82.9836) (width 0.2) (layer "F.Cu") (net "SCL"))
 (segment (start 147.11 124.92) (end 147.39 124.92) (width 0.2) (layer "B.Cu") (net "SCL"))
 (segment (start 134.69 112.5) (end 147.11 124.92) (width 0.2) (layer "B.Cu") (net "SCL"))
 (segment (start 131.315 137.62) (end 132.15 137.62) (width 0.2) (layer "F.Cu") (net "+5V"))
 (segment (start 167.8298 78.3602) (end 166.27 79.92) (width 0.2) (layer "F.Cu") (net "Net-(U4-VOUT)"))
 (segment (start 167.8298 71.9723) (end 167.8298 78.3602) (width 0.2) (layer "F.Cu") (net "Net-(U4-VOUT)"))
 (segment (start 167.22 71.3625) (end 167.8298 71.9723) (width 0.2) (layer "F.Cu") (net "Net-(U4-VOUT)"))
 (segment (start 142.035 81) (end 142.035 86.735) (width 0.2) (layer "B.Cu") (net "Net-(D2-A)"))
 (segment (start 142.035 86.735) (end 140.77 88) (width 0.2) (layer "B.Cu") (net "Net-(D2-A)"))
 (segment (start 160.15 122.96) (end 160.15 120.42) (width 0.2) (layer "F.Cu") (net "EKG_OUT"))
 (segment (start 165.495 128.305) (end 160.15 122.96) (width 0.2) (layer "F.Cu") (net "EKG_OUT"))
 (segment (start 165.495 138.5) (end 165.495 128.305) (width 0.2) (layer "F.Cu") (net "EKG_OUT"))
 (segment (start 167.77 122.96) (end 167.77 125.5) (width 0.2) (layer "F.Cu") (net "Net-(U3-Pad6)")))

